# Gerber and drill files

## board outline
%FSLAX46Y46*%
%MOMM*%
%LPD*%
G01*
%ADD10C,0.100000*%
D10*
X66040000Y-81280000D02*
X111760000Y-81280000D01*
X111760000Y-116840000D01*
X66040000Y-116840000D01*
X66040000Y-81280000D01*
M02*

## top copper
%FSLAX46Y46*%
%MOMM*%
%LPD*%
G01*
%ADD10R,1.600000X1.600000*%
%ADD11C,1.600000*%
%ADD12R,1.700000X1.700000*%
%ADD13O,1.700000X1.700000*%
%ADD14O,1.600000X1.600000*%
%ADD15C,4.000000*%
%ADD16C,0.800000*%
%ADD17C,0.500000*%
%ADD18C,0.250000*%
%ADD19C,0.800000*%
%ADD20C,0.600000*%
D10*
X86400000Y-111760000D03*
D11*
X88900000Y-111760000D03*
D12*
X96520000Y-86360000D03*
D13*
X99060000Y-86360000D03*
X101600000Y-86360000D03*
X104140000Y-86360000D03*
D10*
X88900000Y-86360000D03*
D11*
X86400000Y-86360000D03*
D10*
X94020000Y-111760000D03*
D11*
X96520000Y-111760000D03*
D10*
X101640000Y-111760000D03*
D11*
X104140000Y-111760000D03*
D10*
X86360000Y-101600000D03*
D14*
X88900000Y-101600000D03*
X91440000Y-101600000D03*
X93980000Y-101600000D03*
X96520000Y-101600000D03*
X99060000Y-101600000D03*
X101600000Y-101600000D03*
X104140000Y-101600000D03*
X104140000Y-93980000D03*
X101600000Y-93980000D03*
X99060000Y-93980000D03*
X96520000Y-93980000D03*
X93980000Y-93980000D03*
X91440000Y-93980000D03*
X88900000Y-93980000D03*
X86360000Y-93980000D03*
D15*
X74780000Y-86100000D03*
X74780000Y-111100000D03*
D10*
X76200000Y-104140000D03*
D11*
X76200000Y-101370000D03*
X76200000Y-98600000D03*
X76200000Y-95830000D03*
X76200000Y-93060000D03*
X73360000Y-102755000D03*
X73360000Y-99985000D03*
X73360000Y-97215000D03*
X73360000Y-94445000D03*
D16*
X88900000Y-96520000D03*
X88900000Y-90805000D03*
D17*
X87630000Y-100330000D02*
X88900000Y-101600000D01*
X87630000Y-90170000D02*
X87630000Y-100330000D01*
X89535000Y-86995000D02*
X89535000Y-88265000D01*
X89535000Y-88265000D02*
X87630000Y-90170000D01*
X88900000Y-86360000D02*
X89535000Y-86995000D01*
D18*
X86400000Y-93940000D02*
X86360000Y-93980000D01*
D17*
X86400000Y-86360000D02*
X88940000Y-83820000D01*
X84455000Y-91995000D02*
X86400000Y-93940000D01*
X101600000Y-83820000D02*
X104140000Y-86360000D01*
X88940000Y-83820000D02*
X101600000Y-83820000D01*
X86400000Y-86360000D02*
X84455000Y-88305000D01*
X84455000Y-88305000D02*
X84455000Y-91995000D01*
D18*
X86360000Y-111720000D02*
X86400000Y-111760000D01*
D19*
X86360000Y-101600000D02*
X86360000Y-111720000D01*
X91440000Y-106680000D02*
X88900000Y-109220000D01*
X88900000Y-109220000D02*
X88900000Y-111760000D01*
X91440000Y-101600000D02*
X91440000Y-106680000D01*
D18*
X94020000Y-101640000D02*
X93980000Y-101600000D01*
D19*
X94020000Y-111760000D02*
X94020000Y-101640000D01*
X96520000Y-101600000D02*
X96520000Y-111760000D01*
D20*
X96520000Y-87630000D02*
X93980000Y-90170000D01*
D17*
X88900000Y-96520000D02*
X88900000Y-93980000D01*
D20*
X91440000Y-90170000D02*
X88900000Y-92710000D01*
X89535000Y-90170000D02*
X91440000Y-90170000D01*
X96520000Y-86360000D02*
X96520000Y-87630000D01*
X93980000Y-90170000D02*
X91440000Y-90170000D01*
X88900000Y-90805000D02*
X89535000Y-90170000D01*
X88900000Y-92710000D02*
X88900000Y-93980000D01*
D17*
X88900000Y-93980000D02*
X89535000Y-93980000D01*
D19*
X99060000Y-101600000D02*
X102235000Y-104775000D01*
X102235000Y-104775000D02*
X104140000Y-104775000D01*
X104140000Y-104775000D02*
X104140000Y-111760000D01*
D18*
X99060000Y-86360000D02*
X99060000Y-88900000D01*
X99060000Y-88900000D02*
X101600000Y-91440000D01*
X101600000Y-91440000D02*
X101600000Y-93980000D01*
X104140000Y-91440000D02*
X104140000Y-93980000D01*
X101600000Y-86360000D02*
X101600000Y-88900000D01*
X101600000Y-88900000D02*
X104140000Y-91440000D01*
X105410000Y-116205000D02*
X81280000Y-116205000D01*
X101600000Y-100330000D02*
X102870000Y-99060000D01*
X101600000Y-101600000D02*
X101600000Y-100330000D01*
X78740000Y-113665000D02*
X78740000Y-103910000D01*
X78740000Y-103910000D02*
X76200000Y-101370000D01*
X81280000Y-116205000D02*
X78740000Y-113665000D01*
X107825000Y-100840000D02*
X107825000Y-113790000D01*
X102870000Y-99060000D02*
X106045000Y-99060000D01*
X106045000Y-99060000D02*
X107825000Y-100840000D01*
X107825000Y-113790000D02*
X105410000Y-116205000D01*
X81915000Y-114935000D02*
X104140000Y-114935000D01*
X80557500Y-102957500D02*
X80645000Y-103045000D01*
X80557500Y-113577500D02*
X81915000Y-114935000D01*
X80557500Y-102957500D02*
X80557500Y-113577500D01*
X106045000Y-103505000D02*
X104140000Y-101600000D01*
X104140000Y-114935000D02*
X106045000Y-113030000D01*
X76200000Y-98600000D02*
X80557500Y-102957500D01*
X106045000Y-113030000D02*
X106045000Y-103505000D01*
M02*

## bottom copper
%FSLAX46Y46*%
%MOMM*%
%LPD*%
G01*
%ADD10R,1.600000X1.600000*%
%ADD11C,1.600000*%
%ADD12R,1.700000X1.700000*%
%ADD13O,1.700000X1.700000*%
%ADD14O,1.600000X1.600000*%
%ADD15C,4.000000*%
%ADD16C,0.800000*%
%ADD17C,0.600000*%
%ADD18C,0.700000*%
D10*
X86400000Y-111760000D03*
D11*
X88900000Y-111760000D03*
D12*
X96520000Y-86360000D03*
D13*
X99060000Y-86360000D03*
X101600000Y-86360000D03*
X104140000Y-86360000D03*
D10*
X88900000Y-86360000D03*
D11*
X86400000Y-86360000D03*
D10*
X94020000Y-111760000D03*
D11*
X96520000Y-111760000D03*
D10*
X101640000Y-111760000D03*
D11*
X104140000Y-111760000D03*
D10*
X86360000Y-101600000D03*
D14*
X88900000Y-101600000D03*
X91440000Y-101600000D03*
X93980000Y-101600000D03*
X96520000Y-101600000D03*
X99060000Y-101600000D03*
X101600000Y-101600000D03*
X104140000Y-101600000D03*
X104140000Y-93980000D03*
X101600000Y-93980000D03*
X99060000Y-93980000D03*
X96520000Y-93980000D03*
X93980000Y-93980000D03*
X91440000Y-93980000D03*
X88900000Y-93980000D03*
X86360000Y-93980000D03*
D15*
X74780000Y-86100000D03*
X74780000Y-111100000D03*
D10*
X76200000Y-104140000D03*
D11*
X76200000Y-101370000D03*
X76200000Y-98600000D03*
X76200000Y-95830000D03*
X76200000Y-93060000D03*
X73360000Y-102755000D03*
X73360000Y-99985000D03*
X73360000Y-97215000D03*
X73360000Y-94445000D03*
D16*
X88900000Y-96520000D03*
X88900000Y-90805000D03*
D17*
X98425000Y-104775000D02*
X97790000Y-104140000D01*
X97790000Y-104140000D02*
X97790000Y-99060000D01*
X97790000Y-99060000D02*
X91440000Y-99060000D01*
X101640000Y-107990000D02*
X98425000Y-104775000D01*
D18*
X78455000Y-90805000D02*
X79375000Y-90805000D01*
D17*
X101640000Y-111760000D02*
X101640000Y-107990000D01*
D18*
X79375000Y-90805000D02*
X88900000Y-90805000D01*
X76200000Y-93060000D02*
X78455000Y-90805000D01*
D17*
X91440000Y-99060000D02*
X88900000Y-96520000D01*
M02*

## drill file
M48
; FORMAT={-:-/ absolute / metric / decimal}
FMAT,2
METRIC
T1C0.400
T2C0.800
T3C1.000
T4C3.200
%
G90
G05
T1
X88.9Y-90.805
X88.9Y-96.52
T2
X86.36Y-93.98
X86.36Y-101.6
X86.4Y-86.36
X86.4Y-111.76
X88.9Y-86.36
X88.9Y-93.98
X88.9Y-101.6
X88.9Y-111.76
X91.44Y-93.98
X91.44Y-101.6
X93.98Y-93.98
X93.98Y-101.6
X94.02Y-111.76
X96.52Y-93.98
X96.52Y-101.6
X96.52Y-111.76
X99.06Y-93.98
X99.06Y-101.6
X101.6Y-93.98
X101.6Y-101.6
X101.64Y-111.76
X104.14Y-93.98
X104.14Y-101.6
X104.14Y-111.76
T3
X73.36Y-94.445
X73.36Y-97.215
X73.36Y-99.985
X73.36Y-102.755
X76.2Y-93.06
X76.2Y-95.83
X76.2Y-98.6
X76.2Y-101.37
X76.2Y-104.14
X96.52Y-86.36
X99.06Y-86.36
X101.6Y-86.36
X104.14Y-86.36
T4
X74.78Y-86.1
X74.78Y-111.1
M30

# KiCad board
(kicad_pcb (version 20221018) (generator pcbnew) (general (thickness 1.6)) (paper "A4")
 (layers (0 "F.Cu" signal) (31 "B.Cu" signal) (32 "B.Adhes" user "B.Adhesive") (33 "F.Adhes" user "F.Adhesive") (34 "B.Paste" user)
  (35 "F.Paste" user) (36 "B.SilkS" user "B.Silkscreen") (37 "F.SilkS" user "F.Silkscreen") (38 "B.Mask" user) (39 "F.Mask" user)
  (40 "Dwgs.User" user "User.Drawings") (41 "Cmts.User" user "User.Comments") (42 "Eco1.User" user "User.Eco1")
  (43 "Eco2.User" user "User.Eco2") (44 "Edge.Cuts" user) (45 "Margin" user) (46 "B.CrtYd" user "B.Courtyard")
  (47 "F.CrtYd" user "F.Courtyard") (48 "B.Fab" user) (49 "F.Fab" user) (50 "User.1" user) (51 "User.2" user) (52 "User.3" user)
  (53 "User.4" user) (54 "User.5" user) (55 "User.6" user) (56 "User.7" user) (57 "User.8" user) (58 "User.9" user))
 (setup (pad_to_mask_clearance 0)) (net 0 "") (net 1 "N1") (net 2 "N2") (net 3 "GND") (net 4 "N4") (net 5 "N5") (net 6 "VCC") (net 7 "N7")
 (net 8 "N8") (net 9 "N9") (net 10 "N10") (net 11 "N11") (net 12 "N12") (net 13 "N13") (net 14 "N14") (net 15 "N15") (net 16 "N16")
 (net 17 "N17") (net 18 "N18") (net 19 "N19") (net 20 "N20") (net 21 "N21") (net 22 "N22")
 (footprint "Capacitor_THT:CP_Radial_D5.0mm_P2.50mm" (layer "F.Cu") (at 86.4 111.76)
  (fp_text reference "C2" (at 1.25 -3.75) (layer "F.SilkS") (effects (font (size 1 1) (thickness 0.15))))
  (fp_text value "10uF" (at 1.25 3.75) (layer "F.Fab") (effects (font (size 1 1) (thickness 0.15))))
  (pad "1" thru_hole rect (at 0 0) (size 1.6 1.6) (drill 0.8) (layers "*.Cu" "*.Mask") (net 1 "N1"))
  (pad "2" thru_hole circle (at 2.5 0) (size 1.6 1.6) (drill 0.8) (layers "*.Cu" "*.Mask") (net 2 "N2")))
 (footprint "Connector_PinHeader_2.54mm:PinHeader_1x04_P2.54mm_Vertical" (layer "F.Cu") (at 96.52 86.36 90)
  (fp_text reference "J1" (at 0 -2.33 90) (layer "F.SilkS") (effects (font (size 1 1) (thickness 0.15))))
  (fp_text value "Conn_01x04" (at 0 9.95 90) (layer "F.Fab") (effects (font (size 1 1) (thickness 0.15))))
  (pad "1" thru_hole rect (at 0 0 90) (size 1.7 1.7) (drill 1) (layers "*.Cu" "*.Mask") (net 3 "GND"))
  (pad "2" thru_hole oval (at 0 2.54 90) (size 1.7 1.7) (drill 1) (layers "*.Cu" "*.Mask") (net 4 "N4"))
  (pad "3" thru_hole oval (at 0 5.08 90) (size 1.7 1.7) (drill 1) (layers "*.Cu" "*.Mask") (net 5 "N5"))
  (pad "4" thru_hole oval (at 0 7.62 90) (size 1.7 1.7) (drill 1) (layers "*.Cu" "*.Mask") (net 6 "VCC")))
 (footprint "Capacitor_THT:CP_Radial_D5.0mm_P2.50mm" (layer "F.Cu") (at 88.9 86.36 180)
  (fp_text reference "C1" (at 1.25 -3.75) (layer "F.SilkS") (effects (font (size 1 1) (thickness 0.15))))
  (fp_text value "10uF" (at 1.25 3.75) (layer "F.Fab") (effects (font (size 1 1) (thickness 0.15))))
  (pad "1" thru_hole rect (at 0 0 180) (size 1.6 1.6) (drill 0.8) (layers "*.Cu" "*.Mask") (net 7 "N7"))
  (pad "2" thru_hole circle (at 2.5 0 180) (size 1.6 1.6) (drill 0.8) (layers "*.Cu" "*.Mask") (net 6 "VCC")))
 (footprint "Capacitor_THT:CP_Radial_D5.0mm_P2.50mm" (layer "F.Cu") (at 94.02 111.76)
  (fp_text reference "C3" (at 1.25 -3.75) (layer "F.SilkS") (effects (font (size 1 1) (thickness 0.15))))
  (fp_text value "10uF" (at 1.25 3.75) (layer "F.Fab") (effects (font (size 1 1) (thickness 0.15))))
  (pad "1" thru_hole rect (at 0 0) (size 1.6 1.6) (drill 0.8) (layers "*.Cu" "*.Mask") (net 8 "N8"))
  (pad "2" thru_hole circle (at 2.5 0) (size 1.6 1.6) (drill 0.8) (layers "*.Cu" "*.Mask") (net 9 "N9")))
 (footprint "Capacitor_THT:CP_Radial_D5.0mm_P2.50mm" (layer "F.Cu") (at 101.64 111.76)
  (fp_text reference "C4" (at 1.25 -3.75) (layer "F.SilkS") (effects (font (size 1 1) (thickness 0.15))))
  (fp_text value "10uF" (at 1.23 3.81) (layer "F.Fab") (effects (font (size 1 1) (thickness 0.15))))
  (pad "1" thru_hole rect (at 0 0) (size 1.6 1.6) (drill 0.8) (layers "*.Cu" "*.Mask") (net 3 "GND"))
  (pad "2" thru_hole circle (at 2.5 0) (size 1.6 1.6) (drill 0.8) (layers "*.Cu" "*.Mask") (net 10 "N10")))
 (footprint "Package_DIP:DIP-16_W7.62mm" (layer "F.Cu") (at 86.36 101.6 90)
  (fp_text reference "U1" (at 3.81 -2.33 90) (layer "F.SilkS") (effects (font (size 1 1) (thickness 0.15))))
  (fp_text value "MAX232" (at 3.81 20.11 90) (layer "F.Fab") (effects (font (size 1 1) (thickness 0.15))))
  (pad "1" thru_hole rect (at 0 0 90) (size 1.6 1.6) (drill 0.8) (layers "*.Cu" "*.Mask") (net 1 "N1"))
  (pad "2" thru_hole oval (at 0 2.54 90) (size 1.6 1.6) (drill 0.8) (layers "*.Cu" "*.Mask") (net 7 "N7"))
  (pad "3" thru_hole oval (at 0 5.08 90) (size 1.6 1.6) (drill 0.8) (layers "*.Cu" "*.Mask") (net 2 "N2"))
  (pad "4" thru_hole oval (at 0 7.62 90) (size 1.6 1.6) (drill 0.8) (layers "*.Cu" "*.Mask") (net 8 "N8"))
  (pad "5" thru_hole oval (at 0 10.16 90) (size 1.6 1.6) (drill 0.8) (layers "*.Cu" "*.Mask") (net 9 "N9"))
  (pad "6" thru_hole oval (at 0 12.7 90) (size 1.6 1.6) (drill 0.8) (layers "*.Cu" "*.Mask") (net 10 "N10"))
  (pad "7" thru_hole oval (at 0 15.24 90) (size 1.6 1.6) (drill 0.8) (layers "*.Cu" "*.Mask") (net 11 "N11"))
  (pad "8" thru_hole oval (at 0 17.78 90) (size 1.6 1.6) (drill 0.8) (layers "*.Cu" "*.Mask") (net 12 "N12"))
  (pad "9" thru_hole oval (at 7.62 17.78 90) (size 1.6 1.6) (drill 0.8) (layers "*.Cu" "*.Mask") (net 5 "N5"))
  (pad "10" thru_hole oval (at 7.62 15.24 90) (size 1.6 1.6) (drill 0.8) (layers "*.Cu" "*.Mask") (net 4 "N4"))
  (pad "11" thru_hole oval (at 7.62 12.7 90) (size 1.6 1.6) (drill 0.8) (layers "*.Cu" "*.Mask") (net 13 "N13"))
  (pad "12" thru_hole oval (at 7.62 10.16 90) (size 1.6 1.6) (drill 0.8) (layers "*.Cu" "*.Mask") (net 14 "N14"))
  (pad "13" thru_hole oval (at 7.62 7.62 90) (size 1.6 1.6) (drill 0.8) (layers "*.Cu" "*.Mask") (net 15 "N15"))
  (pad "14" thru_hole oval (at 7.62 5.08 90) (size 1.6 1.6) (drill 0.8) (layers "*.Cu" "*.Mask") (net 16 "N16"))
  (pad "15" thru_hole oval (at 7.62 2.54 90) (size 1.6 1.6) (drill 0.8) (layers "*.Cu" "*.Mask") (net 3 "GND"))
  (pad "16" thru_hole oval (at 7.62 0 90) (size 1.6 1.6) (drill 0.8) (layers "*.Cu" "*.Mask") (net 6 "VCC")))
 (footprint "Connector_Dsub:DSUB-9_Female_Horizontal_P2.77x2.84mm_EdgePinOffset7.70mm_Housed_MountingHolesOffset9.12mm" (layer "F.Cu")
  (at 76.2 104.14 -90)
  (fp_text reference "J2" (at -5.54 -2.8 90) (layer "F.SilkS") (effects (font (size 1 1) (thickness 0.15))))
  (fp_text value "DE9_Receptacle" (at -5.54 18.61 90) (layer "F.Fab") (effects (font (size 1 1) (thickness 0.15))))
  (pad "0" thru_hole circle (at -18.04 1.42 270) (size 4 4) (drill 3.2) (layers "*.Cu" "*.Mask"))
  (pad "0" thru_hole circle (at 6.96 1.42 270) (size 4 4) (drill 3.2) (layers "*.Cu" "*.Mask"))
  (pad "1" thru_hole rect (at 0 0 270) (size 1.6 1.6) (drill 1) (layers "*.Cu" "*.Mask") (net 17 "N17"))
  (pad "2" thru_hole circle (at -2.77 0 270) (size 1.6 1.6) (drill 1) (layers "*.Cu" "*.Mask") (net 11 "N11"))
  (pad "3" thru_hole circle (at -5.54 0 270) (size 1.6 1.6) (drill 1) (layers "*.Cu" "*.Mask") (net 12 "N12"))
  (pad "4" thru_hole circle (at -8.31 0 270) (size 1.6 1.6) (drill 1) (layers "*.Cu" "*.Mask") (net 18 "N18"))
  (pad "5" thru_hole circle (at -11.08 0 270) (size 1.6 1.6) (drill 1) (layers "*.Cu" "*.Mask") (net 3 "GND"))
  (pad "6" thru_hole circle (at -1.385 2.84 270) (size 1.6 1.6) (drill 1) (layers "*.Cu" "*.Mask") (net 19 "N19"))
  (pad "7" thru_hole circle (at -4.155 2.84 270) (size 1.6 1.6) (drill 1) (layers "*.Cu" "*.Mask") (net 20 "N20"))
  (pad "8" thru_hole circle (at -6.925 2.84 270) (size 1.6 1.6) (drill 1) (layers "*.Cu" "*.Mask") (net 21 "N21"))
  (pad "9" thru_hole circle (at -9.695 2.84 270) (size 1.6 1.6) (drill 1) (layers "*.Cu" "*.Mask") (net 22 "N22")))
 (gr_rect (start 66.04 81.28) (end 111.76 116.84) (stroke (width 0.1) (type default)) (fill none) (layer "Edge.Cuts"))
 (segment (start 87.63 100.33) (end 88.9 101.6) (width 0.5) (layer "F.Cu") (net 7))
 (segment (start 87.63 90.17) (end 87.63 100.33) (width 0.5) (layer "F.Cu") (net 7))
 (segment (start 89.535 86.995) (end 89.535 88.265) (width 0.5) (layer "F.Cu") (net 7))
 (segment (start 89.535 88.265) (end 87.63 90.17) (width 0.5) (layer "F.Cu") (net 7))
 (segment (start 88.9 86.36) (end 89.535 86.995) (width 0.5) (layer "F.Cu") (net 7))
 (segment (start 86.4 93.94) (end 86.36 93.98) (width 0.25) (layer "F.Cu") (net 6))
 (segment (start 86.4 86.36) (end 88.94 83.82) (width 0.5) (layer "F.Cu") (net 6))
 (segment (start 84.455 91.995) (end 86.4 93.94) (width 0.5) (layer "F.Cu") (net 6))
 (segment (start 101.6 83.82) (end 104.14 86.36) (width 0.5) (layer "F.Cu") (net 6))
 (segment (start 88.94 83.82) (end 101.6 83.82) (width 0.5) (layer "F.Cu") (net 6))
 (segment (start 86.4 86.36) (end 84.455 88.305) (width 0.5) (layer "F.Cu") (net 6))
 (segment (start 84.455 88.305) (end 84.455 91.995) (width 0.5) (layer "F.Cu") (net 6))
 (segment (start 86.36 111.72) (end 86.4 111.76) (width 0.25) (layer "F.Cu") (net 1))
 (segment (start 86.36 101.6) (end 86.36 111.72) (width 0.8) (layer "F.Cu") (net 1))
 (segment (start 91.44 106.68) (end 88.9 109.22) (width 0.8) (layer "F.Cu") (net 2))
 (segment (start 88.9 109.22) (end 88.9 111.76) (width 0.8) (layer "F.Cu") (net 2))
 (segment (start 91.44 101.6) (end 91.44 106.68) (width 0.8) (layer "F.Cu") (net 2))
 (segment (start 94.02 101.64) (end 93.98 101.6) (width 0.25) (layer "F.Cu") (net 8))
 (segment (start 94.02 111.76) (end 94.02 101.64) (width 0.8) (layer "F.Cu") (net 8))
 (segment (start 96.52 101.6) (end 96.52 111.76) (width 0.8) (layer "F.Cu") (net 9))
 (segment (start 96.52 87.63) (end 93.98 90.17) (width 0.6) (layer "F.Cu") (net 3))
 (segment (start 88.9 96.52) (end 88.9 93.98) (width 0.5) (layer "F.Cu") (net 3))
 (segment (start 91.44 90.17) (end 88.9 92.71) (width 0.6) (layer "F.Cu") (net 3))
 (segment (start 89.535 90.17) (end 91.44 90.17) (width 0.6) (layer "F.Cu") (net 3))
 (segment (start 96.52 86.36) (end 96.52 87.63) (width 0.6) (layer "F.Cu") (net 3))
 (segment (start 93.98 90.17) (end 91.44 90.17) (width 0.6) (layer "F.Cu") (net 3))
 (segment (start 88.9 90.805) (end 89.535 90.17) (width 0.6) (layer "F.Cu") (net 3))
 (segment (start 88.9 92.71) (end 88.9 93.98) (width 0.6) (layer "F.Cu") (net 3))
 (segment (start 88.9 93.98) (end 89.535 93.98) (width 0.5) (layer "F.Cu") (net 3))
 (via (at 88.9 96.52) (size 0.8) (drill 0.4) (layers "F.Cu" "B.Cu") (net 3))
 (via (at 88.9 90.805) (size 0.8) (drill 0.4) (layers "F.Cu" "B.Cu") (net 3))
 (segment (start 98.425 104.775) (end 97.79 104.14) (width 0.6) (layer "B.Cu") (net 3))
 (segment (start 97.79 104.14) (end 97.79 99.06) (width 0.6) (layer "B.Cu") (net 3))
 (segment (start 97.79 99.06) (end 91.44 99.06) (width 0.6) (layer "B.Cu") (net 3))
 (segment (start 101.64 107.99) (end 98.425 104.775) (width 0.6) (layer "B.Cu") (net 3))
 (segment (start 78.455 90.805) (end 79.375 90.805) (width 0.7) (layer "B.Cu") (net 3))
 (segment (start 101.64 111.76) (end 101.64 107.99) (width 0.6) (layer "B.Cu") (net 3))
 (segment (start 79.375 90.805) (end 88.9 90.805) (width 0.7) (layer "B.Cu") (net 3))
 (segment (start 76.2 93.06) (end 78.455 90.805) (width 0.7) (layer "B.Cu") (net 3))
 (segment (start 91.44 99.06) (end 88.9 96.52) (width 0.6) (layer "B.Cu") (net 3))
 (segment (start 99.06 101.6) (end 102.235 104.775) (width 0.8) (layer "F.Cu") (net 10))
 (segment (start 102.235 104.775) (end 104.14 104.775) (width 0.8) (layer "F.Cu") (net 10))
 (segment (start 104.14 104.775) (end 104.14 111.76) (width 0.8) (layer "F.Cu") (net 10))
 (segment (start 99.06 86.36) (end 99.06 88.9) (width 0.25) (layer "F.Cu") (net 4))
 (segment (start 99.06 88.9) (end 101.6 91.44) (width 0.25) (layer "F.Cu") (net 4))
 (segment (start 101.6 91.44) (end 101.6 93.98) (width 0.25) (layer "F.Cu") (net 4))
 (segment (start 104.14 91.44) (end 104.14 93.98) (width 0.25) (layer "F.Cu") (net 5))
 (segment (start 101.6 86.36) (end 101.6 88.9) (width 0.25) (layer "F.Cu") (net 5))
 (segment (start 101.6 88.9) (end 104.14 91.44) (width 0.25) (layer "F.Cu") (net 5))
 (segment (start 105.41 116.205) (end 81.28 116.205) (width 0.25) (layer "F.Cu") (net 11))
 (segment (start 101.6 100.33) (end 102.87 99.06) (width 0.25) (layer "F.Cu") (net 11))
 (segment (start 101.6 101.6) (end 101.6 100.33) (width 0.25) (layer "F.Cu") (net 11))
 (segment (start 78.74 113.665) (end 78.74 103.91) (width 0.25) (layer "F.Cu") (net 11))
 (segment (start 78.74 103.91) (end 76.2 101.37) (width 0.25) (layer "F.Cu") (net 11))
 (segment (start 81.28 116.205) (end 78.74 113.665) (width 0.25) (layer "F.Cu") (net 11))
 (segment (start 107.825 100.84) (end 107.825 113.79) (width 0.25) (layer "F.Cu") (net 11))
 (segment (start 102.87 99.06) (end 106.045 99.06) (width 0.25) (layer "F.Cu") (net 11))
 (segment (start 106.045 99.06) (end 107.825 100.84) (width 0.25) (layer "F.Cu") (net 11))
 (segment (start 107.825 113.79) (end 105.41 116.205) (width 0.25) (layer "F.Cu") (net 11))
 (segment (start 81.915 114.935) (end 104.14 114.935) (width 0.25) (layer "F.Cu") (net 12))
 (segment (start 80.5575 102.9575) (end 80.645 103.045) (width 0.25) (layer "F.Cu") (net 12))
 (segment (start 80.5575 113.5775) (end 81.915 114.935) (width 0.25) (layer "F.Cu") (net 12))
 (segment (start 80.5575 102.9575) (end 80.5575 113.5775) (width 0.25) (layer "F.Cu") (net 12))
 (segment (start 106.045 103.505) (end 104.14 101.6) (width 0.25) (layer "F.Cu") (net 12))
 (segment (start 104.14 114.935) (end 106.045 113.03) (width 0.25) (layer "F.Cu") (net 12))
 (segment (start 76.2 98.6) (end 80.5575 102.9575) (width 0.25) (layer "F.Cu") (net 12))
 (segment (start 106.045 113.03) (end 106.045 103.505) (width 0.25) (layer "F.Cu") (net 12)))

